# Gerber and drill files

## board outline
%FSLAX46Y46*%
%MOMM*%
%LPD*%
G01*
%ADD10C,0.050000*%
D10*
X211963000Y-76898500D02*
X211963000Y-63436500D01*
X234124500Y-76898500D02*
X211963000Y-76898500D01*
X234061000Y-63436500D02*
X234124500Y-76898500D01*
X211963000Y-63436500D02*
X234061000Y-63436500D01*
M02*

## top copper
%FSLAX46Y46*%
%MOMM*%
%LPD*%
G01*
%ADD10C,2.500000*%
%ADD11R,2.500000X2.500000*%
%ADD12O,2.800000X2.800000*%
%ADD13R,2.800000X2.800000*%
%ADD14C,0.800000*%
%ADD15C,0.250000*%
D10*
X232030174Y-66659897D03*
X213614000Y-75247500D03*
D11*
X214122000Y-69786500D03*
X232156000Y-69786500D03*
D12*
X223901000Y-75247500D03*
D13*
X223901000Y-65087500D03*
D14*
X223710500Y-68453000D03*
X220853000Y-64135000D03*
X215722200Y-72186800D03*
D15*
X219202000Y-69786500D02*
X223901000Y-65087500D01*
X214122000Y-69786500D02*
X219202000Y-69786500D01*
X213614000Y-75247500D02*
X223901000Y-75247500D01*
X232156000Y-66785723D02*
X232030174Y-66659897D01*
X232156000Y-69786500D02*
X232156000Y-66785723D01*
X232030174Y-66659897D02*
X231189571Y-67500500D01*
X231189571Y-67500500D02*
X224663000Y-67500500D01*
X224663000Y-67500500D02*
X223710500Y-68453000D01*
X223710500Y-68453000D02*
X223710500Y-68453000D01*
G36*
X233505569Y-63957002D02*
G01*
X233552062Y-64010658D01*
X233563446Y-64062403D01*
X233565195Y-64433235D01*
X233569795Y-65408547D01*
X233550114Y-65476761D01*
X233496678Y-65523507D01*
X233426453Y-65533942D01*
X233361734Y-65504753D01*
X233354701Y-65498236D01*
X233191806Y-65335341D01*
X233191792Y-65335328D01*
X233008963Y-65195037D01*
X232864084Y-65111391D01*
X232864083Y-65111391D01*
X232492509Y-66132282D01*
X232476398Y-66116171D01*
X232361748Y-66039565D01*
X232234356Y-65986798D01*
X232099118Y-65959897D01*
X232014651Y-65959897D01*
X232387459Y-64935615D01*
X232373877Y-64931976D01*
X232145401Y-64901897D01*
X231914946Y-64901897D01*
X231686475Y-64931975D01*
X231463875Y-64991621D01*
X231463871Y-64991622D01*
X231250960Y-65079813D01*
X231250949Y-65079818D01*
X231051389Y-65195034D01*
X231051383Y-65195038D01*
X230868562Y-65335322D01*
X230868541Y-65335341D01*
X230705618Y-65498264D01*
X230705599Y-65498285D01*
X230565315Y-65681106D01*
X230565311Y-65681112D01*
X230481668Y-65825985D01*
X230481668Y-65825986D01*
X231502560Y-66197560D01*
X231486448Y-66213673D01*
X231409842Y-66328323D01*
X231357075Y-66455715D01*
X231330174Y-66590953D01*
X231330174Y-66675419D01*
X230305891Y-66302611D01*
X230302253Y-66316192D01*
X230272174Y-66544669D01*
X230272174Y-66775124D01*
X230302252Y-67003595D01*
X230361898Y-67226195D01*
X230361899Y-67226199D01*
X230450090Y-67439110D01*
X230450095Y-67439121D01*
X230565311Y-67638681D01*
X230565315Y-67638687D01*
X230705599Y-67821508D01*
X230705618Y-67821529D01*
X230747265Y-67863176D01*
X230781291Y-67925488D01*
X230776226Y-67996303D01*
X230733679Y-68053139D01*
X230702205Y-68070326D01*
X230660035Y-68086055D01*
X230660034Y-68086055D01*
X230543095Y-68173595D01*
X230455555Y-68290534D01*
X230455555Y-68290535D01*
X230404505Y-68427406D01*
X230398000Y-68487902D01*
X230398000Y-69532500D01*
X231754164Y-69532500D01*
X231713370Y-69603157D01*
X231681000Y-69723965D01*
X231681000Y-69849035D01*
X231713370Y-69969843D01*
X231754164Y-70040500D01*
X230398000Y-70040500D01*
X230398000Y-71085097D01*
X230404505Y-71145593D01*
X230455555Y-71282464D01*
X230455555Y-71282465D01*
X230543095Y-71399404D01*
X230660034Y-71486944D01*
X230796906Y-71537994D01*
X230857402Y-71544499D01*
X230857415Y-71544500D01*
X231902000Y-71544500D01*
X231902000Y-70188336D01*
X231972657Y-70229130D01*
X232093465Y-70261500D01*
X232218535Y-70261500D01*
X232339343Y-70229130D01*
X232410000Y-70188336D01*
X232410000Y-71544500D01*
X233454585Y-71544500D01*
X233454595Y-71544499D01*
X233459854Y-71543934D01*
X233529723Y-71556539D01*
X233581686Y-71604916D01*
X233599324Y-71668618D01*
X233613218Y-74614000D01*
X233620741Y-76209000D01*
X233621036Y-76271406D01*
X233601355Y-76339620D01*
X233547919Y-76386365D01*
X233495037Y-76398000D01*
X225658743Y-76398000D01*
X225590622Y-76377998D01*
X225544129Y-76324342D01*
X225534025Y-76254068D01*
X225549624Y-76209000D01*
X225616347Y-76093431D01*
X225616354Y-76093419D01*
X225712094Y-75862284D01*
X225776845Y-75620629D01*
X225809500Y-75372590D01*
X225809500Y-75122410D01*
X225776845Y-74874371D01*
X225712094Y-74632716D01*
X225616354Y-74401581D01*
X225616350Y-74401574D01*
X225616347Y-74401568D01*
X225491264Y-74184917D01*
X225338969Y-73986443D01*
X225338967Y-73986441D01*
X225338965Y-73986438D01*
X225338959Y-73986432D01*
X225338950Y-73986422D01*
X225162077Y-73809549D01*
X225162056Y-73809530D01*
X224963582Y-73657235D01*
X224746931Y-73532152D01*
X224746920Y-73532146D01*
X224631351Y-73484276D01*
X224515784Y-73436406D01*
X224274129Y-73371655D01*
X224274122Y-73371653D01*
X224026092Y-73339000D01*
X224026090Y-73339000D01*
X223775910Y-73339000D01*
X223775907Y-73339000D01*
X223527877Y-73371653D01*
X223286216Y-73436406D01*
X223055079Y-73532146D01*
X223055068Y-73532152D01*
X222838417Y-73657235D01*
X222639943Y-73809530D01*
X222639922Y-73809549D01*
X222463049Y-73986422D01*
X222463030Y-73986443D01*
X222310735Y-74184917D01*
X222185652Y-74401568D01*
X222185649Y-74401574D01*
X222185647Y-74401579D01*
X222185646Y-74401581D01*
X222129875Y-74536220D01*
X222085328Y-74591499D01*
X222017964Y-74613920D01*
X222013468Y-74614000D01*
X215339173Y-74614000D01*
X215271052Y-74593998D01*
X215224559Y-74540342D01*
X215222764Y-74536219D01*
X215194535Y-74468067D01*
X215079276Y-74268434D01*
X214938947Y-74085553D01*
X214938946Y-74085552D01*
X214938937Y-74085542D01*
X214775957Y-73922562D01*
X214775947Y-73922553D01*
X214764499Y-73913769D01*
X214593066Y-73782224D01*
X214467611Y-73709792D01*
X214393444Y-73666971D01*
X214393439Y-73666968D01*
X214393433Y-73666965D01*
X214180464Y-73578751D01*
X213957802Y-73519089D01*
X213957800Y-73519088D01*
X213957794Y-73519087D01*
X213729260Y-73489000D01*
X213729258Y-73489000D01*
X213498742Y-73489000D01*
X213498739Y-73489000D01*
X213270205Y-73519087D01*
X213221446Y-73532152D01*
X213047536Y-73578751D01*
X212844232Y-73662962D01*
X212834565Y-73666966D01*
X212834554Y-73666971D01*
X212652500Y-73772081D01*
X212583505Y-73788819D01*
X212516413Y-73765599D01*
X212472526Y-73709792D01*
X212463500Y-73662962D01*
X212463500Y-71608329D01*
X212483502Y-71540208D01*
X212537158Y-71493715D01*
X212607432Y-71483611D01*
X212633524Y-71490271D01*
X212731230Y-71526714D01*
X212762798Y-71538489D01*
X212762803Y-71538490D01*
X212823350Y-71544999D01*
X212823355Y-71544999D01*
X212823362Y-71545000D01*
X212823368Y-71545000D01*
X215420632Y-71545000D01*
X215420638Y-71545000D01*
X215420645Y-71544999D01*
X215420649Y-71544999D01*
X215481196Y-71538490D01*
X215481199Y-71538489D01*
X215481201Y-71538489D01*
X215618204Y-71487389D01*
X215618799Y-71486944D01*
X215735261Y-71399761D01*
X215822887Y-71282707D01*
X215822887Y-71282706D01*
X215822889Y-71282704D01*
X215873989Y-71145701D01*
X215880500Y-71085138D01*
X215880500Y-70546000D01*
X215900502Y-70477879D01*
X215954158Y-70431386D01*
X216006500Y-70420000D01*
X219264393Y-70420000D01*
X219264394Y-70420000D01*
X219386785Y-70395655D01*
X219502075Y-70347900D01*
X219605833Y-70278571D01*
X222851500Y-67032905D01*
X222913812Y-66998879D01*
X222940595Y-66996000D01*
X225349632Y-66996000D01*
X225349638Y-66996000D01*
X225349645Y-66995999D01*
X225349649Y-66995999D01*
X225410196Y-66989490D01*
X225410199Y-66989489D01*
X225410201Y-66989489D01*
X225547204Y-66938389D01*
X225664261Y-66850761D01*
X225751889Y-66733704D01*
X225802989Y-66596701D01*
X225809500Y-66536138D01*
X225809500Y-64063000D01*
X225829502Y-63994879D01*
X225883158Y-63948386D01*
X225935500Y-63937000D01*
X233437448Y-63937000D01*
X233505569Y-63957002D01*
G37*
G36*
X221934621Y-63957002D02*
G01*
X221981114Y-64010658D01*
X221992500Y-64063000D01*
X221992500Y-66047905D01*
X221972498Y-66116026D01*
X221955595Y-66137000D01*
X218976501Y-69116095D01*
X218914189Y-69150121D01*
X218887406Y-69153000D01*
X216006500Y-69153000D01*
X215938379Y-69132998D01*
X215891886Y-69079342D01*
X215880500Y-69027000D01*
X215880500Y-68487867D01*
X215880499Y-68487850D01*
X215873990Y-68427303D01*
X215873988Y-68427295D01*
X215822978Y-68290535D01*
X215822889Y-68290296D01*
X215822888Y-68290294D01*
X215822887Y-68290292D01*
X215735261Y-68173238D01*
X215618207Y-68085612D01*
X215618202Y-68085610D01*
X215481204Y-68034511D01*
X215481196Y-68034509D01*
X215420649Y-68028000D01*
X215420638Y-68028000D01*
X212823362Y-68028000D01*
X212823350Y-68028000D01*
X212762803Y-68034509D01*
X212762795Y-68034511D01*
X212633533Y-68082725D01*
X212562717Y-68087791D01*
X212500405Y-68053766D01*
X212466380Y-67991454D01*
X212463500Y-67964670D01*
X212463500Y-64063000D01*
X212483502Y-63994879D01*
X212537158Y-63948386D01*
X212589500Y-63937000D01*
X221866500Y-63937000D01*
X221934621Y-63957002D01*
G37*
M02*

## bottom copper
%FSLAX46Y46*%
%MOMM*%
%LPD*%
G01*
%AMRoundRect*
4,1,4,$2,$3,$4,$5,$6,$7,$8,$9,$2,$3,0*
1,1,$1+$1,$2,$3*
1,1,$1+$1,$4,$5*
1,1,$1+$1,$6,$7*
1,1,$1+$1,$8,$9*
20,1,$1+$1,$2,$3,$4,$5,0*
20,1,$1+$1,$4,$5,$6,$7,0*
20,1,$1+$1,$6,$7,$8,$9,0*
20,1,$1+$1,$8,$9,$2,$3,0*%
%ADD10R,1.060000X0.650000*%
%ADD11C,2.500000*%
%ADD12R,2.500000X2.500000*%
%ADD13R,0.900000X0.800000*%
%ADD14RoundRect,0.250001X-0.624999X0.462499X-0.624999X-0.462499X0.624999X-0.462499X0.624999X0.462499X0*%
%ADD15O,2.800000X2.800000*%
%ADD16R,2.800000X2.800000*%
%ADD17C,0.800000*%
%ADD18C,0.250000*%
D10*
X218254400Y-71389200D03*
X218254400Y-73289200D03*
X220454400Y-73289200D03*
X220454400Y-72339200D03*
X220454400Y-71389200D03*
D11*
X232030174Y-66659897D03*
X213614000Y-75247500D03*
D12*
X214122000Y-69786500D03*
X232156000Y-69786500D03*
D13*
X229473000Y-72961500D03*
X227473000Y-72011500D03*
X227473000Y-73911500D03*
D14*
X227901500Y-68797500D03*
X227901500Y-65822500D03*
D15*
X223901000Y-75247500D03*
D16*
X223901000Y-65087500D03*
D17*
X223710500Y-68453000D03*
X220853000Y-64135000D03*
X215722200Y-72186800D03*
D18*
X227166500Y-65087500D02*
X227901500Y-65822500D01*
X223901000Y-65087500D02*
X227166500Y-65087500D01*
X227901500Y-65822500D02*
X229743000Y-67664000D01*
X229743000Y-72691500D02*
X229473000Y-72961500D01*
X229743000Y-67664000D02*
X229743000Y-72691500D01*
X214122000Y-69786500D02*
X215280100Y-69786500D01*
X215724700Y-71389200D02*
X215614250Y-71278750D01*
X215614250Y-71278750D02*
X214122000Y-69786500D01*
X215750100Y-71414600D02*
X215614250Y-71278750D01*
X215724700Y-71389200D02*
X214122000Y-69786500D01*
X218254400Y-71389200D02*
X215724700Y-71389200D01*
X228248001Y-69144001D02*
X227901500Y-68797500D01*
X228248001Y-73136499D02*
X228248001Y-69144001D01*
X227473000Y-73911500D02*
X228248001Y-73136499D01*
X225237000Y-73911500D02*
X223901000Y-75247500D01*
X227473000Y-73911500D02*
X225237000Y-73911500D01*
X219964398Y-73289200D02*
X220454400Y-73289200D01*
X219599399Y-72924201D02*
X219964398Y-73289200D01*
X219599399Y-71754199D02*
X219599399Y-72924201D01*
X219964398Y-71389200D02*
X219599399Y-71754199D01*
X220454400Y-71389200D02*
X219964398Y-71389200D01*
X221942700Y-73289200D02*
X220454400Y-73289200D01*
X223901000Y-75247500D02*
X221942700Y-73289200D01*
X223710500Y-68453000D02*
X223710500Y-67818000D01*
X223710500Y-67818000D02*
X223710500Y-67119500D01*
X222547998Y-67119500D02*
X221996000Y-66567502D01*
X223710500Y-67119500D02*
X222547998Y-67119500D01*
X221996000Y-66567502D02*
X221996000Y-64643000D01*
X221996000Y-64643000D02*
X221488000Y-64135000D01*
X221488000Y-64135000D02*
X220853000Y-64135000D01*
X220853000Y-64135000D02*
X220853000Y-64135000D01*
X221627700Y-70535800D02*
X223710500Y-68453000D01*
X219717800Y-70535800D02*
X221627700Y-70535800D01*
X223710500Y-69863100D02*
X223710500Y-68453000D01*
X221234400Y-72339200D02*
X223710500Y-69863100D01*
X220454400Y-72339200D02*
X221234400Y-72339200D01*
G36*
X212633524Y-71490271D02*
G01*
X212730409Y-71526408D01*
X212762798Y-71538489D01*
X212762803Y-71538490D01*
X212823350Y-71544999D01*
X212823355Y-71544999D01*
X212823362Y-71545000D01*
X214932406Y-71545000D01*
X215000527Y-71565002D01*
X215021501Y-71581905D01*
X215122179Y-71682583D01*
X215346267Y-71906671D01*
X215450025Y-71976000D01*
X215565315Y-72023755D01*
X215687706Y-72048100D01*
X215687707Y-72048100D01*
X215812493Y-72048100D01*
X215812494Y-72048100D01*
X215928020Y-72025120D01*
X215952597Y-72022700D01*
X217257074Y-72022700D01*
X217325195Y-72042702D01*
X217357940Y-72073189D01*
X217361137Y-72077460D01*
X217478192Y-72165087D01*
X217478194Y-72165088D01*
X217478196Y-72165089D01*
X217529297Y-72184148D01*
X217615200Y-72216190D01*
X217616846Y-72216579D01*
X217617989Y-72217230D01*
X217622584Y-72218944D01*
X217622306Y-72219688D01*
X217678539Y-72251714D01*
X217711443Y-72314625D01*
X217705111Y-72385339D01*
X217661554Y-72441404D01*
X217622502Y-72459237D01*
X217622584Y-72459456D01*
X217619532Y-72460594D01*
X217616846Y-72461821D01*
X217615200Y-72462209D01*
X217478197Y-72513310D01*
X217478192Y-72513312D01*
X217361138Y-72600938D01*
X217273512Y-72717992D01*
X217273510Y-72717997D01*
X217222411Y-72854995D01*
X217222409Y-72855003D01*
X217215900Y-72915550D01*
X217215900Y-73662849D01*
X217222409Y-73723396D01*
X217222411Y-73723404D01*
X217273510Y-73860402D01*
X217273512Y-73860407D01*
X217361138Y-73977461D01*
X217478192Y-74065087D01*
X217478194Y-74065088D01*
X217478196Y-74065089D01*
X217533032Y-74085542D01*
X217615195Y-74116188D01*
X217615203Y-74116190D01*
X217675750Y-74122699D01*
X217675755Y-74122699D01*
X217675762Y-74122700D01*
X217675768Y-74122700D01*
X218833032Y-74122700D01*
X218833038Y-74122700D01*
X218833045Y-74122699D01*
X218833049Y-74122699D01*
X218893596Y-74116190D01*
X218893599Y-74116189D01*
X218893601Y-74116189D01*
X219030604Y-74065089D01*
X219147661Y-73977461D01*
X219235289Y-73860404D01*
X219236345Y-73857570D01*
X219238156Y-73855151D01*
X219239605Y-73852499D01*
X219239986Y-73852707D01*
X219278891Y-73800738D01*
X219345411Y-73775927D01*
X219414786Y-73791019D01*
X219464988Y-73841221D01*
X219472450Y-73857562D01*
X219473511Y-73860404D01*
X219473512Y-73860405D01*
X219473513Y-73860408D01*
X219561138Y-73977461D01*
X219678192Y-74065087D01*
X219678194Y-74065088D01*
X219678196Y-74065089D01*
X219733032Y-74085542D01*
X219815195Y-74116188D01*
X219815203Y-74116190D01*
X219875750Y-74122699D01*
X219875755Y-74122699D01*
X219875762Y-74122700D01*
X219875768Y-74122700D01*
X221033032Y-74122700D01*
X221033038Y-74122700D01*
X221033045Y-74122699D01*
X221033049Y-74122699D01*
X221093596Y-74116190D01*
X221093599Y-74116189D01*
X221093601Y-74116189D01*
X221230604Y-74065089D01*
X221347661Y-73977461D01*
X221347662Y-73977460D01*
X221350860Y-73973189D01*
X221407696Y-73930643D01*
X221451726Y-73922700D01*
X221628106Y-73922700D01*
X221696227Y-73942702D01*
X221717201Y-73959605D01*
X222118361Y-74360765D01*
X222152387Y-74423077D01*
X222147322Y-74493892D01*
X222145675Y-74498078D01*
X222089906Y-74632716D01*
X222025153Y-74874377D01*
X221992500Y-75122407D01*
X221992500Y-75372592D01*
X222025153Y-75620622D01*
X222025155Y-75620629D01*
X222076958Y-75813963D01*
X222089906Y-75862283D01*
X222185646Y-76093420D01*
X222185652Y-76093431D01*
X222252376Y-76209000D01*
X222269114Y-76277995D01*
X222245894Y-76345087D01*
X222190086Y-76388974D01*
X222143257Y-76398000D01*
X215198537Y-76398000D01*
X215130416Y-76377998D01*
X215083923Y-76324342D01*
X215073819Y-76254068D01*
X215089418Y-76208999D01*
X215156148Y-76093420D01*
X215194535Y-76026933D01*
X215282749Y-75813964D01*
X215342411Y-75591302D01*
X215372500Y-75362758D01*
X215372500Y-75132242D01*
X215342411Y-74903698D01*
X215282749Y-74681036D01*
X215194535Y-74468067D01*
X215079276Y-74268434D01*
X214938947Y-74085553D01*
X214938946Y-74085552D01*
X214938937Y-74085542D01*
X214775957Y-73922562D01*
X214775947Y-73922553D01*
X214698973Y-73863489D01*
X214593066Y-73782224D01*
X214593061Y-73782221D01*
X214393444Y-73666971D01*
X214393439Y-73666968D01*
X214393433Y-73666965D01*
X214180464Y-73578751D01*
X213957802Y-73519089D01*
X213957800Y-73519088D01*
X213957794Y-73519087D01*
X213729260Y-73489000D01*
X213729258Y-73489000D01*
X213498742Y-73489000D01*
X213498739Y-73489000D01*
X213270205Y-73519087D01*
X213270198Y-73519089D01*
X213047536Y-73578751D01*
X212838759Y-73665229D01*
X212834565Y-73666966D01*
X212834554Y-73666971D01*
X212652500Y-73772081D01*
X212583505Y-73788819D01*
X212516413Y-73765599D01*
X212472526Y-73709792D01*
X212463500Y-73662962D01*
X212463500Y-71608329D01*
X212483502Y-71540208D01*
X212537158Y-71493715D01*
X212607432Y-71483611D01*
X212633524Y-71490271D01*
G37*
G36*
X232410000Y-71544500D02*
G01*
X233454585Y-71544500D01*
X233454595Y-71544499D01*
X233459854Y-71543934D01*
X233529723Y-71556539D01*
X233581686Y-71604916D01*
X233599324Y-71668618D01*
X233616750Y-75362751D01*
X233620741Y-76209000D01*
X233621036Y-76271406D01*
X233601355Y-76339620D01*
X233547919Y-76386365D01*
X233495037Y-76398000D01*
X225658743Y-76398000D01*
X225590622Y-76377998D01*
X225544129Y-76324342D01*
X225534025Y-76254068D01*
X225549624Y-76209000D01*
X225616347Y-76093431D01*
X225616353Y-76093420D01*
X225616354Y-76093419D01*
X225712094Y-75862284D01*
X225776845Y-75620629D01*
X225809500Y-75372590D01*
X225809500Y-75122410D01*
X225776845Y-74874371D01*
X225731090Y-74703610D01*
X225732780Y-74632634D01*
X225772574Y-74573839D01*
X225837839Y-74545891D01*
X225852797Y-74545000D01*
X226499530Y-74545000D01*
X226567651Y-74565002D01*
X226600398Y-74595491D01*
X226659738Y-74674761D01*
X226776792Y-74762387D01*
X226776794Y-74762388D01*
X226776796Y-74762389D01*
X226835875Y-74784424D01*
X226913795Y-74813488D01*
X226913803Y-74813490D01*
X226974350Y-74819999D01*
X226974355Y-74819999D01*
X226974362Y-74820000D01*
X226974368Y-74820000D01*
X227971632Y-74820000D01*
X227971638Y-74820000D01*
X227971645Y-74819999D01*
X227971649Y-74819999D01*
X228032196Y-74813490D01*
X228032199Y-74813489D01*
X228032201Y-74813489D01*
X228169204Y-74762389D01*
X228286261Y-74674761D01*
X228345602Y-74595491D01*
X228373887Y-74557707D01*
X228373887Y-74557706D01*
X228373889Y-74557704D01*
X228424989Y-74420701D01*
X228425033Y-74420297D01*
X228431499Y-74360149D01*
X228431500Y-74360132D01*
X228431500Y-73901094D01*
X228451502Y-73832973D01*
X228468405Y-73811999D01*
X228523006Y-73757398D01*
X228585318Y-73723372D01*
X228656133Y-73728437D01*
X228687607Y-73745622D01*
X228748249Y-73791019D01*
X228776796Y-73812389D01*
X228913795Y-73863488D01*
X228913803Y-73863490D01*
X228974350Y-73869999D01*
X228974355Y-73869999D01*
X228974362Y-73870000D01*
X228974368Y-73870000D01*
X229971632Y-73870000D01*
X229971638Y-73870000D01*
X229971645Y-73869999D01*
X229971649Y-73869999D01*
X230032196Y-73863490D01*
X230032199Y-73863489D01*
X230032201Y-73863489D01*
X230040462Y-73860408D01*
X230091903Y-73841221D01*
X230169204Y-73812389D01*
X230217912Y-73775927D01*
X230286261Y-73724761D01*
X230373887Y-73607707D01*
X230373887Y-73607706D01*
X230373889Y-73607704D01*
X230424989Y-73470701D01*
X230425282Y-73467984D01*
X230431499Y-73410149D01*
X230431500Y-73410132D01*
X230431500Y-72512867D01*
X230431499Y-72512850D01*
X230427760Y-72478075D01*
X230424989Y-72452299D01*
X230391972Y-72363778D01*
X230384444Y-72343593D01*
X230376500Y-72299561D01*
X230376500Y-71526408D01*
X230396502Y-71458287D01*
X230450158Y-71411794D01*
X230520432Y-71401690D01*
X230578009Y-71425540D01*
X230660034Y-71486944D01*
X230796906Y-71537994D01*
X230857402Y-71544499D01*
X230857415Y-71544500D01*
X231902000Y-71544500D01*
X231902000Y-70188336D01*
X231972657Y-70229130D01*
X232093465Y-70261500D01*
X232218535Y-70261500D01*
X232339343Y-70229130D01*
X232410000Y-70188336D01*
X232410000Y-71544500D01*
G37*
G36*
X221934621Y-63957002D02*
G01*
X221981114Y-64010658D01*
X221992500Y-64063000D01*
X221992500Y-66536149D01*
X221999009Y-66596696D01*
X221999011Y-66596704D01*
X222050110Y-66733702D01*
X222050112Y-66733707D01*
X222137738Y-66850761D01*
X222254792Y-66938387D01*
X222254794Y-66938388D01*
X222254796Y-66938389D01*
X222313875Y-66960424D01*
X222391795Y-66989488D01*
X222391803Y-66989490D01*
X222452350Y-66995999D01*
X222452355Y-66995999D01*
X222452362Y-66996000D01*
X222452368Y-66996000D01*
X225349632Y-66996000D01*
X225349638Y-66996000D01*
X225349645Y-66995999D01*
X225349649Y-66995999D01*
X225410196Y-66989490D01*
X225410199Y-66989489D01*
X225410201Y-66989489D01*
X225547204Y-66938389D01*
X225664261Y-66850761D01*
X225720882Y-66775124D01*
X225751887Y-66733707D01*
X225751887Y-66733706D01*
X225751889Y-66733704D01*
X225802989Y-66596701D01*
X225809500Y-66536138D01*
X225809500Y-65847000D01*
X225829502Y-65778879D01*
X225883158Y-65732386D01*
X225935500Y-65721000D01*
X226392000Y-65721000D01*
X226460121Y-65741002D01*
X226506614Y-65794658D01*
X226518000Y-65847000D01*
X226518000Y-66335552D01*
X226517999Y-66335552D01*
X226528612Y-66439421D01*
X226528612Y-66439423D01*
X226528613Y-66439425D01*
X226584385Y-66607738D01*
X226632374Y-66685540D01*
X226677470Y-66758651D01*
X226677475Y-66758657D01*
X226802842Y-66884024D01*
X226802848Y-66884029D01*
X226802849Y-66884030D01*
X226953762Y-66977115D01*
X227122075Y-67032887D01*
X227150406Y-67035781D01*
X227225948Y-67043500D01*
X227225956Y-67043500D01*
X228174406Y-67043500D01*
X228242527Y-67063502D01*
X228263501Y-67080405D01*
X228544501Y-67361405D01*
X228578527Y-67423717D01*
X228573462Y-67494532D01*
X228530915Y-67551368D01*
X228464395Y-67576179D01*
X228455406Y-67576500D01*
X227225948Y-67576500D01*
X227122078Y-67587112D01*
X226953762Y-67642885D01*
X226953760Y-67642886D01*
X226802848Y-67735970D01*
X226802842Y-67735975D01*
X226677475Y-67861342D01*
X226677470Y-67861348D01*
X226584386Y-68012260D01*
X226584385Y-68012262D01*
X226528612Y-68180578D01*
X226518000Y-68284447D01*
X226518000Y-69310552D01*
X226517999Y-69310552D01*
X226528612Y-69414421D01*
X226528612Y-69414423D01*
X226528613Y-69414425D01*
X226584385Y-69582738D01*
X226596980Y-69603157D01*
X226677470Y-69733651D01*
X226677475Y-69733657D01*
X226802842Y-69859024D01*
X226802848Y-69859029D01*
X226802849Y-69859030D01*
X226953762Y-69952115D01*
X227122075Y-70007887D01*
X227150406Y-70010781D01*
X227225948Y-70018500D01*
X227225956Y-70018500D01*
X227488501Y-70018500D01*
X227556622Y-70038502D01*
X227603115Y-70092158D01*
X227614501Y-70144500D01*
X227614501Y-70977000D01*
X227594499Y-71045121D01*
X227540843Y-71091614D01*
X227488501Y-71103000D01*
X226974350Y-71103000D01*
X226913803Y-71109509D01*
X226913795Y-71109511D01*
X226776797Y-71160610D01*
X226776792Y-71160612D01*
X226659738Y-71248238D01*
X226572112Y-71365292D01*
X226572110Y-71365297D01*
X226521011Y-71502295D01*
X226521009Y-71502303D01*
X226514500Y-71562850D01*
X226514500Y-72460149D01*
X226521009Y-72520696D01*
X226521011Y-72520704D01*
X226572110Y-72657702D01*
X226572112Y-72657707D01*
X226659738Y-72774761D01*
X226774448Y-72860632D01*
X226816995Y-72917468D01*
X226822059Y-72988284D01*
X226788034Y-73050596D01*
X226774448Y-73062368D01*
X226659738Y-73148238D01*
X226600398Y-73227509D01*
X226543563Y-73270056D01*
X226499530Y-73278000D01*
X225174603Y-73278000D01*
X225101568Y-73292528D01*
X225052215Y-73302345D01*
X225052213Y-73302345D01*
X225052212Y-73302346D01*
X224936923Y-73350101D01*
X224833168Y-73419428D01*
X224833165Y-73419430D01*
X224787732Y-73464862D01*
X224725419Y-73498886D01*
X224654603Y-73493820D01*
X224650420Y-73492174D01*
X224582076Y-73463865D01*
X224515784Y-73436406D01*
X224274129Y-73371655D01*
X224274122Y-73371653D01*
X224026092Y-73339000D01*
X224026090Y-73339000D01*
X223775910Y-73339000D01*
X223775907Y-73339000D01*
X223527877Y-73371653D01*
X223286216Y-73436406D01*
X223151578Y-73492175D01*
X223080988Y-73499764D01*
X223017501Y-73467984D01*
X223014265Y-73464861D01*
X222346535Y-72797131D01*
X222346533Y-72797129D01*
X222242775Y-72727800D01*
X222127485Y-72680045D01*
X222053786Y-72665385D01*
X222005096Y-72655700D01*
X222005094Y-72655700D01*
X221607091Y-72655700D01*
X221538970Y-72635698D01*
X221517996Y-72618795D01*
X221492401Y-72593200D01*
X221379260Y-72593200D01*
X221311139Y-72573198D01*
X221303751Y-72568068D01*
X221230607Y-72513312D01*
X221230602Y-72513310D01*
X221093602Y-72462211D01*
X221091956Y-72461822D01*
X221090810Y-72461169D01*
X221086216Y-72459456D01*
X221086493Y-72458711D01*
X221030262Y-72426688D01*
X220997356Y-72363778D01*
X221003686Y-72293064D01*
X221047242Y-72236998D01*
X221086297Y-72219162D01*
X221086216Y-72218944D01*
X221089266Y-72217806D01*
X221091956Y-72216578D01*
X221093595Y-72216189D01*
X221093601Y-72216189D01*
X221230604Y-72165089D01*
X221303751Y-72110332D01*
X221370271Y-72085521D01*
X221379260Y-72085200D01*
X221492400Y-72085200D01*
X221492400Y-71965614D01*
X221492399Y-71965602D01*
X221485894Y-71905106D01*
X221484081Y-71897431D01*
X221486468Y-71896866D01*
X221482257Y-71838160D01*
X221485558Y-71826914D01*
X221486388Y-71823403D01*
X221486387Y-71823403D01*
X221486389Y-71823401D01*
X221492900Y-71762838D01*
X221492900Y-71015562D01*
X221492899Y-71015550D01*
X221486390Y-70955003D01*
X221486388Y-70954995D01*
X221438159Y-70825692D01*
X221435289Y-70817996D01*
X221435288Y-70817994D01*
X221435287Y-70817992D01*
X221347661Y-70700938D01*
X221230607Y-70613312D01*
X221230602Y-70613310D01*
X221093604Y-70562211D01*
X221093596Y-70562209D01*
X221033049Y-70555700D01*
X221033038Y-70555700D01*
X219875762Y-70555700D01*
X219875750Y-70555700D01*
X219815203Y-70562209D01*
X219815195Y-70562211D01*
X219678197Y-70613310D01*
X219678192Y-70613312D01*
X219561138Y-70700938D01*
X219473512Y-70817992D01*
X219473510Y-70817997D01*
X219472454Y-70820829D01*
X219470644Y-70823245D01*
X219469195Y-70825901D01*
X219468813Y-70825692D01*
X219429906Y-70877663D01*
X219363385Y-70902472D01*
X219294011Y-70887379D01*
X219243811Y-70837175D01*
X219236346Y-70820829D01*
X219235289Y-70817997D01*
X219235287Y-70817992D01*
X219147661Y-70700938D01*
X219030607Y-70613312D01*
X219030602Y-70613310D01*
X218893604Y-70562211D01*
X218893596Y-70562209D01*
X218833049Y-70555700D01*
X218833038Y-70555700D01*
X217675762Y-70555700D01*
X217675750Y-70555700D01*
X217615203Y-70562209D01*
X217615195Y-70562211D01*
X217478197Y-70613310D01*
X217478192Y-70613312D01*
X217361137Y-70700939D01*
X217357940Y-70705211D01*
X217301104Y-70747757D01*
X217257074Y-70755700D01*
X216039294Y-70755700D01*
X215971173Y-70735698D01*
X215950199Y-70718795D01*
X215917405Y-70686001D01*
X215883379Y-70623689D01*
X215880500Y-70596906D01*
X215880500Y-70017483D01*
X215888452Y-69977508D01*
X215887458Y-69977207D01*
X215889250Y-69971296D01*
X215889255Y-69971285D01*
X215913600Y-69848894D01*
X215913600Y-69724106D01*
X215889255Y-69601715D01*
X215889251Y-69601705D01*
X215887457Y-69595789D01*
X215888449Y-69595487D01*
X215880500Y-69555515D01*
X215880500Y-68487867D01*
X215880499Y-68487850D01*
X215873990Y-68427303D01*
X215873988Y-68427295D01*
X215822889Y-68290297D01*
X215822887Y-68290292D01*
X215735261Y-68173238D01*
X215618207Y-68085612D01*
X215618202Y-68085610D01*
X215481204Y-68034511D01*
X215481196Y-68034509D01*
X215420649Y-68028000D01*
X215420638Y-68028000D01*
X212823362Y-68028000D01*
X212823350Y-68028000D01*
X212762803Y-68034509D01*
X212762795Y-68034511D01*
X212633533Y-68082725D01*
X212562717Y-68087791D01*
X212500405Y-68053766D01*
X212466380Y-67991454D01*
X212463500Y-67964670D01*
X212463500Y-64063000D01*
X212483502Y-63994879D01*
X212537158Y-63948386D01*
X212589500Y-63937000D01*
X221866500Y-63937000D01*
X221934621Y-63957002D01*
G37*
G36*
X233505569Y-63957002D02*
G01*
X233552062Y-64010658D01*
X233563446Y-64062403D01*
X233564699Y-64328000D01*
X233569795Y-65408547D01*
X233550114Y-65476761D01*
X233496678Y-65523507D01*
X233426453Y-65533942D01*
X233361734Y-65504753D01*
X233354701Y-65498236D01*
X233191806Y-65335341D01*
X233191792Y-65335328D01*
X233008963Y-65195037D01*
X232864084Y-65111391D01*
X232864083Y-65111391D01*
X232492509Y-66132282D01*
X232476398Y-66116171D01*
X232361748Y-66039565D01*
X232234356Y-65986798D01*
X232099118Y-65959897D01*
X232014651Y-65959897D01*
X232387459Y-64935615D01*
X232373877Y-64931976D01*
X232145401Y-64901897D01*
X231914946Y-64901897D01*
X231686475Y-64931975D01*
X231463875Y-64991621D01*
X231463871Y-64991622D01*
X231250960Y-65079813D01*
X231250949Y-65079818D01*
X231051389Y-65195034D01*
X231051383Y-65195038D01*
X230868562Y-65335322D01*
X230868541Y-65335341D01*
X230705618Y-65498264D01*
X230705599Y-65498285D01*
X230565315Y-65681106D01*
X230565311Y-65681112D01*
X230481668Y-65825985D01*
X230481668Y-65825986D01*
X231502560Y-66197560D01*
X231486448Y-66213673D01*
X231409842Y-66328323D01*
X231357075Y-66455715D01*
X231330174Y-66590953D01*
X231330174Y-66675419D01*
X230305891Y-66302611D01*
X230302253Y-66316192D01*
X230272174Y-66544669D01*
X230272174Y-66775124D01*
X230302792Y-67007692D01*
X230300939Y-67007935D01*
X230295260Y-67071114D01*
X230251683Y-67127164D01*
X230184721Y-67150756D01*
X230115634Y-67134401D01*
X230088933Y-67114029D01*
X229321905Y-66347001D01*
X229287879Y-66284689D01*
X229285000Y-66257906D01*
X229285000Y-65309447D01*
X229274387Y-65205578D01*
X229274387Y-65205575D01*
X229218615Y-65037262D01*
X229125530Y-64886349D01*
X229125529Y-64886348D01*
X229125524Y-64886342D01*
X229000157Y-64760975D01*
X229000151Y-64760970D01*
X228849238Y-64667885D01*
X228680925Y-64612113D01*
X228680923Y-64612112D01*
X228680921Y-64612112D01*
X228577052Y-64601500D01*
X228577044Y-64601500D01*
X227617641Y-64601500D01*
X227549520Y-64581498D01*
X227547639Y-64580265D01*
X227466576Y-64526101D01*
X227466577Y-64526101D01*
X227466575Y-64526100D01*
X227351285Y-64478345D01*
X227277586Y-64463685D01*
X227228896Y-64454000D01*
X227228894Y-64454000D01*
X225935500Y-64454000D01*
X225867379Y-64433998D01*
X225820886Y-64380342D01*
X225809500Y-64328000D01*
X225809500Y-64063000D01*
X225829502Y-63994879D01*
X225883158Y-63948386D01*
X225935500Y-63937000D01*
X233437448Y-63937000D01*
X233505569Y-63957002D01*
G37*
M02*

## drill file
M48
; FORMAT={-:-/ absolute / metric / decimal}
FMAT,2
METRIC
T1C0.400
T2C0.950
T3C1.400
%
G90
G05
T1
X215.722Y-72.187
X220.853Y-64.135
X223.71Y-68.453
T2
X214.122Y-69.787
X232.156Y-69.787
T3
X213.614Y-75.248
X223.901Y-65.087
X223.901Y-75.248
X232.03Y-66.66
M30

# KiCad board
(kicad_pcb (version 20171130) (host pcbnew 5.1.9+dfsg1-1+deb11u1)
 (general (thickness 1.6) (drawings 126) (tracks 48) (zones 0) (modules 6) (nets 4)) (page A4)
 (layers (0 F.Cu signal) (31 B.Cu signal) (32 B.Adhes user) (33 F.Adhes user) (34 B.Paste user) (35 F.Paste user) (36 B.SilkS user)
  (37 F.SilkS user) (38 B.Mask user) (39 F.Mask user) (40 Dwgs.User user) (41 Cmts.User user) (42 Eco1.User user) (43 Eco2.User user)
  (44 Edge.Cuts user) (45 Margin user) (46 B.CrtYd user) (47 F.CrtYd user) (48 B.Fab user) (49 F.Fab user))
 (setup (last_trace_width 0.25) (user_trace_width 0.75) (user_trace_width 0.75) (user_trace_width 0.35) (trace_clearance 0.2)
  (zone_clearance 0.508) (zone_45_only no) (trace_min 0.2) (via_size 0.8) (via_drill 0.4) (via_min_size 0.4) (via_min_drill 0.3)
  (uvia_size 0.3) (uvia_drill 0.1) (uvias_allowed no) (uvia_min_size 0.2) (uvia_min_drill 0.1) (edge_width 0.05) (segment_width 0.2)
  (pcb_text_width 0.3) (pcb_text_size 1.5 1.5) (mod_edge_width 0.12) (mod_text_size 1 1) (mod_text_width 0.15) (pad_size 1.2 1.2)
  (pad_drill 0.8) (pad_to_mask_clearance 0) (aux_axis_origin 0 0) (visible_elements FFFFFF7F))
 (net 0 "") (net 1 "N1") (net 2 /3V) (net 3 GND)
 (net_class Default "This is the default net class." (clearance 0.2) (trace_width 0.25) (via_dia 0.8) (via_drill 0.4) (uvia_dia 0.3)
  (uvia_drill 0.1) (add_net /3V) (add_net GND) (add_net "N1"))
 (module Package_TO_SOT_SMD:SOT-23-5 (layer B.Cu) (at 219.3544 72.3392 180)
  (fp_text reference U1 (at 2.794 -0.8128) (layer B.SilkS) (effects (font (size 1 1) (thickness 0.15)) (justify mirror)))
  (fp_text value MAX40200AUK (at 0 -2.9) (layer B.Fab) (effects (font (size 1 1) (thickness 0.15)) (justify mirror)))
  (pad 5 smd rect (at 1.1 0.95 180) (size 1.06 0.65) (layers B.Cu B.Paste B.Mask) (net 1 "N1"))
  (pad 4 smd rect (at 1.1 -0.95 180) (size 1.06 0.65) (layers B.Cu B.Paste B.Mask))
  (pad 3 smd rect (at -1.1 -0.95 180) (size 1.06 0.65) (layers B.Cu B.Paste B.Mask) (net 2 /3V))
  (pad 2 smd rect (at -1.1 0 180) (size 1.06 0.65) (layers B.Cu B.Paste B.Mask) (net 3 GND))
  (pad 1 smd rect (at -1.1 0.95 180) (size 1.06 0.65) (layers B.Cu B.Paste B.Mask) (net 2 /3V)))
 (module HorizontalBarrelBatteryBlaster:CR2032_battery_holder (layer F.Cu) (at 213.614 75.2475 25)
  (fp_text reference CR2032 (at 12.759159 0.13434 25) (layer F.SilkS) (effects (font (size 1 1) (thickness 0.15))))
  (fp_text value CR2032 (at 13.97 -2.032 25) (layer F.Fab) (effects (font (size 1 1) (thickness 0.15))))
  (pad 2 thru_hole circle (at 20.32 0 25) (size 2.5 2.5) (drill 1.4) (layers *.Cu *.Mask) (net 3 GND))
  (pad 1 thru_hole circle (at 0 0 25) (size 2.5 2.5) (drill 1.4) (layers *.Cu *.Mask) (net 2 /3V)))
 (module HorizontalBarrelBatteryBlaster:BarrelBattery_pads (layer B.Cu) (at 232.156 69.7865 180)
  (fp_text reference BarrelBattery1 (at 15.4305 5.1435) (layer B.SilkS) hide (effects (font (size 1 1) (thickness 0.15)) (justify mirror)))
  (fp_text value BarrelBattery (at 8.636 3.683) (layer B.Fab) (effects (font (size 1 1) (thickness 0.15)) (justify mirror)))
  (pad 1 thru_hole rect (at 18.034 0 180) (size 2.5 2.5) (drill 0.95) (layers *.Cu *.Mask) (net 1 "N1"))
  (pad 2 thru_hole rect (at 0 0 90) (size 2.5 2.5) (drill 0.95) (layers *.Cu *.Mask) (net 3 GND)))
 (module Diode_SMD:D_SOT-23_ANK (layer B.Cu) (at 228.473 72.9615)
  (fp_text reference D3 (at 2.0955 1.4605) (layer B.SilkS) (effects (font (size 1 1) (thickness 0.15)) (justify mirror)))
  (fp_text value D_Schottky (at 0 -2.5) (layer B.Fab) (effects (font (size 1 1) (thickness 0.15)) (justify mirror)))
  (pad 1 smd rect (at 1 0) (size 0.9 0.8) (layers B.Cu B.Paste B.Mask) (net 1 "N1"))
  (pad "" smd rect (at -1 -0.95) (size 0.9 0.8) (layers B.Cu B.Paste B.Mask))
  (pad 2 smd rect (at -1 0.95) (size 0.9 0.8) (layers B.Cu B.Paste B.Mask) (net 2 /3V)))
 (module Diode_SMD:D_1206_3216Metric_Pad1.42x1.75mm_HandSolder (layer B.Cu) (at 227.9015 67.31 270)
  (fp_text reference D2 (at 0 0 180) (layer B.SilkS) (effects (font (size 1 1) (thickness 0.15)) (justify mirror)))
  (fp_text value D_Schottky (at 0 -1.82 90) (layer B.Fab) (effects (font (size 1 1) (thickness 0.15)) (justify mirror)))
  (pad 2 smd roundrect (at 1.4875 0 270) (size 1.425 1.75) (layers B.Cu B.Paste B.Mask) (roundrect_rratio 0.175439) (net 2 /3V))
  (pad 1 smd roundrect (at -1.4875 0 270) (size 1.425 1.75) (layers B.Cu B.Paste B.Mask) (roundrect_rratio 0.175439) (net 1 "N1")))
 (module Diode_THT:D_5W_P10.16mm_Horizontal (layer B.Cu) (at 223.901 65.0875 270)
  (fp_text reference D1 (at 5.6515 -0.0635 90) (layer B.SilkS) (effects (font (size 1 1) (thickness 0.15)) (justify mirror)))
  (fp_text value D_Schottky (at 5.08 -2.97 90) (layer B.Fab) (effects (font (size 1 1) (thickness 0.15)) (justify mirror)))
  (pad 2 thru_hole oval (at 10.16 0 270) (size 2.8 2.8) (drill 1.4) (layers *.Cu *.Mask) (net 2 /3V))
  (pad 1 thru_hole rect (at 0 0 270) (size 2.8 2.8) (drill 1.4) (layers *.Cu *.Mask) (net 1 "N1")))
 (gr_line (start 211.963 76.8985) (end 211.963 63.4365) (layer Edge.Cuts) (width 0.05))
 (gr_line (start 234.1245 76.8985) (end 211.963 76.8985) (layer Edge.Cuts) (width 0.05))
 (gr_line (start 234.061 63.4365) (end 234.1245 76.8985) (layer Edge.Cuts) (width 0.05))
 (gr_line (start 211.963 63.4365) (end 234.061 63.4365) (layer Edge.Cuts) (width 0.05))
 (segment (start 219.202 69.7865) (end 223.901 65.0875) (width 0.25) (layer F.Cu) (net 1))
 (segment (start 214.122 69.7865) (end 219.202 69.7865) (width 0.25) (layer F.Cu) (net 1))
 (segment (start 227.1665 65.0875) (end 227.9015 65.8225) (width 0.25) (layer B.Cu) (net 1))
 (segment (start 223.901 65.0875) (end 227.1665 65.0875) (width 0.25) (layer B.Cu) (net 1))
 (segment (start 227.9015 65.8225) (end 229.743 67.664) (width 0.25) (layer B.Cu) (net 1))
 (segment (start 229.743 72.6915) (end 229.473 72.9615) (width 0.25) (layer B.Cu) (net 1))
 (segment (start 229.743 67.664) (end 229.743 72.6915) (width 0.25) (layer B.Cu) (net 1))
 (segment (start 214.122 69.7865) (end 215.2801 69.7865) (width 0.25) (layer B.Cu) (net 1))
 (segment (start 215.7247 71.3892) (end 215.61425 71.27875) (width 0.25) (layer B.Cu) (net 1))
 (segment (start 215.61425 71.27875) (end 214.122 69.7865) (width 0.25) (layer B.Cu) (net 1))
 (segment (start 215.7501 71.4146) (end 215.61425 71.27875) (width 0.25) (layer B.Cu) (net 1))
 (segment (start 215.7247 71.3892) (end 214.122 69.7865) (width 0.25) (layer B.Cu) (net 1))
 (segment (start 218.2544 71.3892) (end 215.7247 71.3892) (width 0.25) (layer B.Cu) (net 1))
 (segment (start 228.248001 69.144001) (end 227.9015 68.7975) (width 0.25) (layer B.Cu) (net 2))
 (segment (start 228.248001 73.136499) (end 228.248001 69.144001) (width 0.25) (layer B.Cu) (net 2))
 (segment (start 227.473 73.9115) (end 228.248001 73.136499) (width 0.25) (layer B.Cu) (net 2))
 (segment (start 213.614 75.2475) (end 223.901 75.2475) (width 0.25) (layer F.Cu) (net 2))
 (segment (start 225.237 73.9115) (end 223.901 75.2475) (width 0.25) (layer B.Cu) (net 2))
 (segment (start 227.473 73.9115) (end 225.237 73.9115) (width 0.25) (layer B.Cu) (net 2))
 (segment (start 219.964398 73.2892) (end 220.4544 73.2892) (width 0.25) (layer B.Cu) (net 2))
 (segment (start 219.599399 72.924201) (end 219.964398 73.2892) (width 0.25) (layer B.Cu) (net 2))
 (segment (start 219.599399 71.754199) (end 219.599399 72.924201) (width 0.25) (layer B.Cu) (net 2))
 (segment (start 219.964398 71.3892) (end 219.599399 71.754199) (width 0.25) (layer B.Cu) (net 2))
 (segment (start 220.4544 71.3892) (end 219.964398 71.3892) (width 0.25) (layer B.Cu) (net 2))
 (segment (start 221.9427 73.2892) (end 220.4544 73.2892) (width 0.25) (layer B.Cu) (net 2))
 (segment (start 223.901 75.2475) (end 221.9427 73.2892) (width 0.25) (layer B.Cu) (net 2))
 (segment (start 232.156 66.785723) (end 232.030174 66.659897) (width 0.25) (layer F.Cu) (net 3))
 (segment (start 232.156 69.7865) (end 232.156 66.785723) (width 0.25) (layer F.Cu) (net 3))
 (segment (start 232.030174 66.659897) (end 231.189571 67.5005) (width 0.25) (layer F.Cu) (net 3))
 (segment (start 231.189571 67.5005) (end 224.663 67.5005) (width 0.25) (layer F.Cu) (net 3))
 (segment (start 224.663 67.5005) (end 223.7105 68.453) (width 0.25) (layer F.Cu) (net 3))
 (segment (start 223.7105 68.453) (end 223.7105 68.453) (width 0.25) (layer F.Cu) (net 3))
 (via (at 223.7105 68.453) (size 0.8) (drill 0.4) (layers F.Cu B.Cu) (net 3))
 (segment (start 223.7105 68.453) (end 223.7105 67.818) (width 0.25) (layer B.Cu) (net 3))
 (segment (start 223.7105 67.818) (end 223.7105 67.1195) (width 0.25) (layer B.Cu) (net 3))
 (segment (start 222.547998 67.1195) (end 221.996 66.567502) (width 0.25) (layer B.Cu) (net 3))
 (segment (start 223.7105 67.1195) (end 222.547998 67.1195) (width 0.25) (layer B.Cu) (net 3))
 (segment (start 221.996 66.567502) (end 221.996 64.643) (width 0.25) (layer B.Cu) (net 3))
 (segment (start 221.996 64.643) (end 221.488 64.135) (width 0.25) (layer B.Cu) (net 3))
 (segment (start 221.488 64.135) (end 220.853 64.135) (width 0.25) (layer B.Cu) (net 3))
 (segment (start 220.853 64.135) (end 220.853 64.135) (width 0.25) (layer B.Cu) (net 3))
 (via (at 220.853 64.135) (size 0.8) (drill 0.4) (layers F.Cu B.Cu) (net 3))
 (segment (start 221.6277 70.5358) (end 223.7105 68.453) (width 0.25) (layer B.Cu) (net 3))
 (segment (start 219.7178 70.5358) (end 221.6277 70.5358) (width 0.25) (layer B.Cu) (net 3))
 (via (at 215.7222 72.1868) (size 0.8) (drill 0.4) (layers F.Cu B.Cu) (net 3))
 (segment (start 223.7105 69.8631) (end 223.7105 68.453) (width 0.25) (layer B.Cu) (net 3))
 (segment (start 221.2344 72.3392) (end 223.7105 69.8631) (width 0.25) (layer B.Cu) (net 3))
 (segment (start 220.4544 72.3392) (end 221.2344 72.3392) (width 0.25) (layer B.Cu) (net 3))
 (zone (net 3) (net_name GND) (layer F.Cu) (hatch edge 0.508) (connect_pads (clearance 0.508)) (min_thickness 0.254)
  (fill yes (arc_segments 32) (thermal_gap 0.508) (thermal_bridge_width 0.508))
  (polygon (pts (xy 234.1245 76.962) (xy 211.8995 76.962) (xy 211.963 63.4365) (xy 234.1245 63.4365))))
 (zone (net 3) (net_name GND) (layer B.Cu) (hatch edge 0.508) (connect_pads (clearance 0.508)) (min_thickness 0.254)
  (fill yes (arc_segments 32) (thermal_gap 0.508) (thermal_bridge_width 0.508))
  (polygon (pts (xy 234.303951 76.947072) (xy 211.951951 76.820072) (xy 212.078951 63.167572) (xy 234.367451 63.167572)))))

